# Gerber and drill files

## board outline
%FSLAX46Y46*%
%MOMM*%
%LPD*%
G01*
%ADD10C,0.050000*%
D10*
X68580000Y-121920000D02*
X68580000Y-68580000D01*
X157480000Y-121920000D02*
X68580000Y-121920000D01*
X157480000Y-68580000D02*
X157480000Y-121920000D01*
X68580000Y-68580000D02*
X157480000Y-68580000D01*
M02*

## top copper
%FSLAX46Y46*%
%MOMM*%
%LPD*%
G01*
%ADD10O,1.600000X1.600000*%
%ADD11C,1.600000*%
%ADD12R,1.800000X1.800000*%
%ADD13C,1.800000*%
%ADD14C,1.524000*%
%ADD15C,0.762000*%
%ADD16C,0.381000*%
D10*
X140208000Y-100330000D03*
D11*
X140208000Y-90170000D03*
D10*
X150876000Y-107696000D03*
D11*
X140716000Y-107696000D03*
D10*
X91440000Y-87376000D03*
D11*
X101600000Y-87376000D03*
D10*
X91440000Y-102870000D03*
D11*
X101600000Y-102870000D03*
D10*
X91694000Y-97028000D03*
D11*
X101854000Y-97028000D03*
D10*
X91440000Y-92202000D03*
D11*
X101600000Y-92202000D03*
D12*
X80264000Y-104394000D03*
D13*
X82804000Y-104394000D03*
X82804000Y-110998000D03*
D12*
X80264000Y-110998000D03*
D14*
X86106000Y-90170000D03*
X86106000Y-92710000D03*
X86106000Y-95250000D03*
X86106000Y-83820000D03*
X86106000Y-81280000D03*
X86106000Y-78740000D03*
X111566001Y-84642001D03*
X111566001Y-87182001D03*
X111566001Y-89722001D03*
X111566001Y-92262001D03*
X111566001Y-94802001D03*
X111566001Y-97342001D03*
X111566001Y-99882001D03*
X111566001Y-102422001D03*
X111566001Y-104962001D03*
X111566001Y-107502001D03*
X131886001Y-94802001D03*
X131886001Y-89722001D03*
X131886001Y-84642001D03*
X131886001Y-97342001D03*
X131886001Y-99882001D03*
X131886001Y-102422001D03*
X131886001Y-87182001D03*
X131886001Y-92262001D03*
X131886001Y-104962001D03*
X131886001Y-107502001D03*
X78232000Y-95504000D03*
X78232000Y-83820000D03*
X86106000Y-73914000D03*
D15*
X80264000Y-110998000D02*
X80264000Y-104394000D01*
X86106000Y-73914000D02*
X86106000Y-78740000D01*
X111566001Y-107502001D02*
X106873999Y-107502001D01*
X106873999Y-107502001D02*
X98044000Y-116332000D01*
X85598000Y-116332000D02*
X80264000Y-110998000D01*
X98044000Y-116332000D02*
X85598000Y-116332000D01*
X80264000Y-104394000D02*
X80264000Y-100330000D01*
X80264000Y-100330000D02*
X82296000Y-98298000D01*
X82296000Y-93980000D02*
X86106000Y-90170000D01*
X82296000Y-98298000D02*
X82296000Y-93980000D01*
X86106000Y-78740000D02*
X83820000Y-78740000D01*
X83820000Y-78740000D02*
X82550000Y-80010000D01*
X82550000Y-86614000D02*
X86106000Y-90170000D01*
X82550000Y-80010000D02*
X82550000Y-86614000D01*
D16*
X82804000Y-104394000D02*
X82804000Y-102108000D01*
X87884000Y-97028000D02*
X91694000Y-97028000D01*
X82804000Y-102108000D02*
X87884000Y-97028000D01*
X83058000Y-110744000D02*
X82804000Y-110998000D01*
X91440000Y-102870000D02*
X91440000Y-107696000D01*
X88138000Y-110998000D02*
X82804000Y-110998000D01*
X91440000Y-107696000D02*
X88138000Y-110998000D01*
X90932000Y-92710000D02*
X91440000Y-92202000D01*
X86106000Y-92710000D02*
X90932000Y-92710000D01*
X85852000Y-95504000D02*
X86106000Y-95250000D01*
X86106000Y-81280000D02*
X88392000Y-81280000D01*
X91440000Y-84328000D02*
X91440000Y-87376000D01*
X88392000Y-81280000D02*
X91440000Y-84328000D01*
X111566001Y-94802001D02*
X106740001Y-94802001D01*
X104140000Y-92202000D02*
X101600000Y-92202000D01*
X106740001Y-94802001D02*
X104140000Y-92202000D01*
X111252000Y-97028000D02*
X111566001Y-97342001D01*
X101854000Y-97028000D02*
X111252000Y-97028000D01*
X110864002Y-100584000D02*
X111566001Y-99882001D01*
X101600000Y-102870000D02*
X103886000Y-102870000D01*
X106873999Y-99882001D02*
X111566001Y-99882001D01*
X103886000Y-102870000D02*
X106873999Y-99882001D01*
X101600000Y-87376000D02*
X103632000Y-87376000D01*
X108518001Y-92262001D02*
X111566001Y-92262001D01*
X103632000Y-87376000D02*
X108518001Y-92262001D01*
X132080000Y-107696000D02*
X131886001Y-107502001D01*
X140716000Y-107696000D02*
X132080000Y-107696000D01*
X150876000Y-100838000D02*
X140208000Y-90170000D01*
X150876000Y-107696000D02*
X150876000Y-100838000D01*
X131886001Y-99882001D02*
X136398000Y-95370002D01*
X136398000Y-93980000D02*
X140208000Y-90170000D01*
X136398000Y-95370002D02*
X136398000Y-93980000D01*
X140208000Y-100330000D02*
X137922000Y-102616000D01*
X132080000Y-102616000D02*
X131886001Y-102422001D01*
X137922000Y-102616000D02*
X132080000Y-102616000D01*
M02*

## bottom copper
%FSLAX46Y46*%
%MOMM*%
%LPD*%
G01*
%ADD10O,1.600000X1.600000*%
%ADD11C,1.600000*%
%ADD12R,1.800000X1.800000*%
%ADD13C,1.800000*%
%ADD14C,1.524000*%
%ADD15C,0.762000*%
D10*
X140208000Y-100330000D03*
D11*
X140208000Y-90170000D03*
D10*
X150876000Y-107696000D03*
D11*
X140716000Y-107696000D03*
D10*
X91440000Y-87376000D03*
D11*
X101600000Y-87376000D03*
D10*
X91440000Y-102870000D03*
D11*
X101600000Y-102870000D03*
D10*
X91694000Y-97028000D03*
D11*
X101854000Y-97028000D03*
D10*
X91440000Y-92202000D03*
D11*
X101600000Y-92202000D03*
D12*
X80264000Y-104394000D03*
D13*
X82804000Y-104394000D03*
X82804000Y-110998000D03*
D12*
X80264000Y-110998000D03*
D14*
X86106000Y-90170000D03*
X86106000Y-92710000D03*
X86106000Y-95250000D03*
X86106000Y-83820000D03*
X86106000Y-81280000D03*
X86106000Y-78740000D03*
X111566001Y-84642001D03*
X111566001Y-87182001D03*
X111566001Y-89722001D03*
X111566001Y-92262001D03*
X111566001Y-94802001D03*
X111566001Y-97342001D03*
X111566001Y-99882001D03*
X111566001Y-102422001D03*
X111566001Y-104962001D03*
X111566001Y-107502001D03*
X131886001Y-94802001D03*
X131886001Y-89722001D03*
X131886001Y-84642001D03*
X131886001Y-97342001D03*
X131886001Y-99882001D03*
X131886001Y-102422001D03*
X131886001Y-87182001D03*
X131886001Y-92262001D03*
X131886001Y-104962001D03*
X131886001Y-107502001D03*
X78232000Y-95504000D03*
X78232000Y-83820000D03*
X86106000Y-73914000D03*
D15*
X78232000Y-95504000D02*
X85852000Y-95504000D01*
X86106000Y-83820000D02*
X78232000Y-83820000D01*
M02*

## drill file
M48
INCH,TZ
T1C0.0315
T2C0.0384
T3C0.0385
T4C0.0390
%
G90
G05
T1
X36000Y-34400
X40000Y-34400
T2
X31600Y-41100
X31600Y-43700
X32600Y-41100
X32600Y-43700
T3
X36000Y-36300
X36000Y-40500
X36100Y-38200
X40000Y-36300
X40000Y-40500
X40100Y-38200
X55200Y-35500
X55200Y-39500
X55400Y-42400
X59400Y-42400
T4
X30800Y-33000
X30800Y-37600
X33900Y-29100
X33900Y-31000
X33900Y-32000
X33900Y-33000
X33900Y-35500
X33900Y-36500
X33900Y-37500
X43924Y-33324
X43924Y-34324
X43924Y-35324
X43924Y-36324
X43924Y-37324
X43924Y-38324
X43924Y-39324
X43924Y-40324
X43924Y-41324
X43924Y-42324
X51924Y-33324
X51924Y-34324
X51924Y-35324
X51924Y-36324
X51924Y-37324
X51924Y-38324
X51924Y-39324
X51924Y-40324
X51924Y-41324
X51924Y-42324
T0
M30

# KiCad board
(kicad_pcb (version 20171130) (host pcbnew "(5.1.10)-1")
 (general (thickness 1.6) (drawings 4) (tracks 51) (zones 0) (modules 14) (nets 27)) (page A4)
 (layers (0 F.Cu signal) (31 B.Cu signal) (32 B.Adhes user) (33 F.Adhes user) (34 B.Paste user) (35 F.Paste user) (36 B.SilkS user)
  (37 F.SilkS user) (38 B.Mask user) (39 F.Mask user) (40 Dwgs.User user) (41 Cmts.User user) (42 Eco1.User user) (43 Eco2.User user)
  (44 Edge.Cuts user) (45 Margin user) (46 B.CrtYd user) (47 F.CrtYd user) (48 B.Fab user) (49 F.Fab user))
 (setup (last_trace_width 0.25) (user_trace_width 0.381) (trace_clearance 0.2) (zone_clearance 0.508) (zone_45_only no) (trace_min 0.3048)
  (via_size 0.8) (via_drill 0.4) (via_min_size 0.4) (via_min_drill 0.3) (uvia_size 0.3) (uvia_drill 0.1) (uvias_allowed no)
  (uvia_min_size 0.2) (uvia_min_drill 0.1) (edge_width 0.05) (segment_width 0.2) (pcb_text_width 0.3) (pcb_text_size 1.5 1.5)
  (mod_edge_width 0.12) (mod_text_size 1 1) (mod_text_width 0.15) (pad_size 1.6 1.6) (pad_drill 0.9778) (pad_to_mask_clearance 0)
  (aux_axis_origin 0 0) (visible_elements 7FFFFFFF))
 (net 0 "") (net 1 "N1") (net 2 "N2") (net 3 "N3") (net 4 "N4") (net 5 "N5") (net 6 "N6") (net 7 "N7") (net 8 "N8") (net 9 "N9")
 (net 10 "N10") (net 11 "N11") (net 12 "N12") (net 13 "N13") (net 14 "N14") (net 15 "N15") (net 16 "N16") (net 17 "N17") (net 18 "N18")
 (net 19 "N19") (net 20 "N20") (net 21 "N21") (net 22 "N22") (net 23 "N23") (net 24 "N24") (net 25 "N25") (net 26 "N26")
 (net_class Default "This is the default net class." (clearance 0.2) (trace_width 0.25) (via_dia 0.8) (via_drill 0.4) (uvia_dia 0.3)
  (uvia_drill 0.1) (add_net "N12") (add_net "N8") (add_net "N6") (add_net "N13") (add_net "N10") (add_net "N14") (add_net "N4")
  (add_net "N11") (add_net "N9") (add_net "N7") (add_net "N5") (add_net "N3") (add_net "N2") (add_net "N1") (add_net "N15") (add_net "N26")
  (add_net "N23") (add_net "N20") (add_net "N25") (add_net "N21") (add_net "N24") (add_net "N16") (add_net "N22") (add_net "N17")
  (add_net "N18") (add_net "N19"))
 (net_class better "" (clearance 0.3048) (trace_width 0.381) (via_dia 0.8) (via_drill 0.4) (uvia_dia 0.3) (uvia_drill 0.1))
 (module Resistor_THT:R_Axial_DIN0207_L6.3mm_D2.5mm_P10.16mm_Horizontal (layer F.Cu) (at 140.208 90.17 270)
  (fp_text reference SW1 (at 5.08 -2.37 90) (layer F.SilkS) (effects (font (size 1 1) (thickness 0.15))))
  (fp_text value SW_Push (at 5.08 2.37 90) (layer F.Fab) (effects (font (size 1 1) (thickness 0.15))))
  (pad 2 thru_hole oval (at 10.16 0 270) (size 1.6 1.6) (drill 0.9778) (layers *.Cu *.Mask) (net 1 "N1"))
  (pad 1 thru_hole circle (at 0 0 270) (size 1.6 1.6) (drill 0.9778) (layers *.Cu *.Mask) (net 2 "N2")))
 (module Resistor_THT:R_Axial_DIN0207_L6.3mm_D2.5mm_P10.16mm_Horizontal (layer F.Cu) (at 140.716 107.696)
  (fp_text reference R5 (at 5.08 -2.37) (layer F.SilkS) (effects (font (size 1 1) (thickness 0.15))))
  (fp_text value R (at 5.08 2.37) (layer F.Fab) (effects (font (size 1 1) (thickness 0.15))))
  (pad 2 thru_hole oval (at 10.16 0) (size 1.6 1.6) (drill 0.9778) (layers *.Cu *.Mask) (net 2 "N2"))
  (pad 1 thru_hole circle (at 0 0) (size 1.6 1.6) (drill 0.9778) (layers *.Cu *.Mask) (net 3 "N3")))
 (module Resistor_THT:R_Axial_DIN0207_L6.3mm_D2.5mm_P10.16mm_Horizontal (layer F.Cu) (at 101.6 87.376 180)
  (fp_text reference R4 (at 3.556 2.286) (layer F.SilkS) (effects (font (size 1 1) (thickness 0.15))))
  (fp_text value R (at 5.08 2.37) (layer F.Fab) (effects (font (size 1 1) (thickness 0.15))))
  (pad 2 thru_hole oval (at 10.16 0 180) (size 1.6 1.6) (drill 0.8) (layers *.Cu *.Mask) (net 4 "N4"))
  (pad 1 thru_hole circle (at 0 0 180) (size 1.6 1.6) (drill 0.8) (layers *.Cu *.Mask) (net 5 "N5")))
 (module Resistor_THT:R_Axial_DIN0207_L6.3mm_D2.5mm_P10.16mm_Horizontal (layer F.Cu) (at 101.6 102.87 180)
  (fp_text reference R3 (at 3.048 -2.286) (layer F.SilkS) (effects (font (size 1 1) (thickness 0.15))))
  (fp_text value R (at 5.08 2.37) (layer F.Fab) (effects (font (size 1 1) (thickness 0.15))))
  (pad 2 thru_hole oval (at 10.16 0 180) (size 1.6 1.6) (drill 0.9778) (layers *.Cu *.Mask) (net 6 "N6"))
  (pad 1 thru_hole circle (at 0 0 180) (size 1.6 1.6) (drill 0.9778) (layers *.Cu *.Mask) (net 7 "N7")))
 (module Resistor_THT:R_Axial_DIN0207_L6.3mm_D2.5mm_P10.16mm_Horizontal (layer F.Cu) (at 101.854 97.028 180)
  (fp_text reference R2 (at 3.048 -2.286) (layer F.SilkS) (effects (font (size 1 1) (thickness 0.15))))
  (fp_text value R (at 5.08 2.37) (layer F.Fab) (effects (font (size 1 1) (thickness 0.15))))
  (pad 2 thru_hole oval (at 10.16 0 180) (size 1.6 1.6) (drill 0.9778) (layers *.Cu *.Mask) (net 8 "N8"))
  (pad 1 thru_hole circle (at 0 0 180) (size 1.6 1.6) (drill 0.9778) (layers *.Cu *.Mask) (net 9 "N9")))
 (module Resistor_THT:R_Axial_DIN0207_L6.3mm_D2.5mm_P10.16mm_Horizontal (layer F.Cu) (at 101.6 92.202 180)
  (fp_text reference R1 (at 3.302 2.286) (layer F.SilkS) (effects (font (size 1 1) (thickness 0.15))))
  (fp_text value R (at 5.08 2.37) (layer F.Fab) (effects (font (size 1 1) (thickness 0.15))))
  (pad 2 thru_hole oval (at 10.16 0 180) (size 1.6 1.6) (drill 0.9778) (layers *.Cu *.Mask) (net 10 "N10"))
  (pad 1 thru_hole circle (at 0 0 180) (size 1.6 1.6) (drill 0.9778) (layers *.Cu *.Mask) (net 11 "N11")))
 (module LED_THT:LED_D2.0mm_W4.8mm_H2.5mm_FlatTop (layer F.Cu) (at 80.264 104.394)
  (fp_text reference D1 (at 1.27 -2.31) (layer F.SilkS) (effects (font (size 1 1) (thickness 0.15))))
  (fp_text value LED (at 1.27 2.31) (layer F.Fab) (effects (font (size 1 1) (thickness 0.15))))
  (pad 1 thru_hole rect (at 0 0) (size 1.8 1.8) (drill 0.9762) (layers *.Cu *.Mask) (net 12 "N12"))
  (pad 2 thru_hole circle (at 2.54 0) (size 1.8 1.8) (drill 0.9762) (layers *.Cu *.Mask) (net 8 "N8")))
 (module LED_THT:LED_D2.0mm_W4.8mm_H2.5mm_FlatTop (layer F.Cu) (at 80.264 110.998)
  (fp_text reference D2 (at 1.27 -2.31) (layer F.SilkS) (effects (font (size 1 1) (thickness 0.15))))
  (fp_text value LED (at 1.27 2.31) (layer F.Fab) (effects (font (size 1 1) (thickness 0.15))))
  (pad 2 thru_hole circle (at 2.54 0) (size 1.8 1.8) (drill 0.9762) (layers *.Cu *.Mask) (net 6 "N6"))
  (pad 1 thru_hole rect (at 0 0) (size 1.8 1.8) (drill 0.9762) (layers *.Cu *.Mask) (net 12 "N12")))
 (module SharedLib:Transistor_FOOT (layer F.Cu) (at 86.106 92.71 90)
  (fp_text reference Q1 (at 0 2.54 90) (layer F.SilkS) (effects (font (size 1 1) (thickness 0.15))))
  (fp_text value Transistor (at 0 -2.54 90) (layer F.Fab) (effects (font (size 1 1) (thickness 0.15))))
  (pad 3 thru_hole circle (at 2.54 0 90) (size 1.524 1.524) (drill 0.9906) (layers *.Cu *.Mask) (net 12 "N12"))
  (pad 2 thru_hole circle (at 0 0 90) (size 1.524 1.524) (drill 0.9906) (layers *.Cu *.Mask) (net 10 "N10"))
  (pad 1 thru_hole circle (at -2.54 0 90) (size 1.524 1.524) (drill 0.9906) (layers *.Cu *.Mask) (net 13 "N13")))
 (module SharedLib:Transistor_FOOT (layer F.Cu) (at 86.106 81.28 90)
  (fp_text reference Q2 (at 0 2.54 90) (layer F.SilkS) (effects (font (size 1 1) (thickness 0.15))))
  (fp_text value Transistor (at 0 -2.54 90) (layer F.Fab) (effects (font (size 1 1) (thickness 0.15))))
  (pad 1 thru_hole circle (at -2.54 0 90) (size 1.524 1.524) (drill 0.9906) (layers *.Cu *.Mask) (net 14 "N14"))
  (pad 2 thru_hole circle (at 0 0 90) (size 1.524 1.524) (drill 0.9906) (layers *.Cu *.Mask) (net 4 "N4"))
  (pad 3 thru_hole circle (at 2.54 0 90) (size 1.524 1.524) (drill 0.9906) (layers *.Cu *.Mask) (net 12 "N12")))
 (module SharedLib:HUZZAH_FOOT (layer F.Cu) (at 121.726001 96.072001)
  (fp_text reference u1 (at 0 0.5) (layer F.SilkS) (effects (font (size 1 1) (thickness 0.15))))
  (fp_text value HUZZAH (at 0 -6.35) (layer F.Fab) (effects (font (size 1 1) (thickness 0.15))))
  (pad 1 thru_hole circle (at -10.16 -11.43) (size 1.524 1.524) (drill 0.9906) (layers *.Cu *.Mask) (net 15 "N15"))
  (pad 2 thru_hole circle (at -10.16 -8.89) (size 1.524 1.524) (drill 0.9906) (layers *.Cu *.Mask) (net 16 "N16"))
  (pad 3 thru_hole circle (at -10.16 -6.35) (size 1.524 1.524) (drill 0.9906) (layers *.Cu *.Mask) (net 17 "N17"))
  (pad 4 thru_hole circle (at -10.16 -3.81) (size 1.524 1.524) (drill 0.9906) (layers *.Cu *.Mask) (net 5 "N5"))
  (pad 5 thru_hole circle (at -10.16 -1.27) (size 1.524 1.524) (drill 0.9906) (layers *.Cu *.Mask) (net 11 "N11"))
  (pad 6 thru_hole circle (at -10.16 1.27) (size 1.524 1.524) (drill 0.9906) (layers *.Cu *.Mask) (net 9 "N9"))
  (pad 7 thru_hole circle (at -10.16 3.81) (size 1.524 1.524) (drill 0.9906) (layers *.Cu *.Mask) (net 7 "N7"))
  (pad 8 thru_hole circle (at -10.16 6.35) (size 1.524 1.524) (drill 0.9906) (layers *.Cu *.Mask) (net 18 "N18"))
  (pad 9 thru_hole circle (at -10.16 8.89) (size 1.524 1.524) (drill 0.9906) (layers *.Cu *.Mask) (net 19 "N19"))
  (pad 10 thru_hole circle (at -10.16 11.43) (size 1.524 1.524) (drill 0.9906) (layers *.Cu *.Mask) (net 12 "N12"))
  (pad 16 thru_hole circle (at 10.16 -1.27) (size 1.524 1.524) (drill 0.9906) (layers *.Cu *.Mask) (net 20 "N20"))
  (pad 18 thru_hole circle (at 10.16 -6.35) (size 1.524 1.524) (drill 0.9906) (layers *.Cu *.Mask) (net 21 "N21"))
  (pad 20 thru_hole circle (at 10.16 -11.43) (size 1.524 1.524) (drill 0.9906) (layers *.Cu *.Mask) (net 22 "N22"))
  (pad 15 thru_hole circle (at 10.16 1.27) (size 1.524 1.524) (drill 0.9906) (layers *.Cu *.Mask) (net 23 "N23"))
  (pad 14 thru_hole circle (at 10.16 3.81) (size 1.524 1.524) (drill 0.9906) (layers *.Cu *.Mask) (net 2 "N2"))
  (pad 13 thru_hole circle (at 10.16 6.35) (size 1.524 1.524) (drill 0.9906) (layers *.Cu *.Mask) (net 1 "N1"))
  (pad 19 thru_hole circle (at 10.16 -8.89) (size 1.524 1.524) (drill 0.9906) (layers *.Cu *.Mask) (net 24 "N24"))
  (pad 17 thru_hole circle (at 10.16 -3.81) (size 1.524 1.524) (drill 0.9906) (layers *.Cu *.Mask) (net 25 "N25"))
  (pad 12 thru_hole circle (at 10.16 8.89) (size 1.524 1.524) (drill 0.9906) (layers *.Cu *.Mask) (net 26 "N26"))
  (pad 11 thru_hole circle (at 10.16 11.43) (size 1.524 1.524) (drill 0.9906) (layers *.Cu *.Mask) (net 3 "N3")))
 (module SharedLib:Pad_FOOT (layer F.Cu) (at 78.232 95.504)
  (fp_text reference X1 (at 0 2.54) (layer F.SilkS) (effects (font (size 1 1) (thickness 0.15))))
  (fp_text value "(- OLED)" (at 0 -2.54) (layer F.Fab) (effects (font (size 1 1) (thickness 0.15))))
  (pad 1 thru_hole circle (at 0 0) (size 1.524 1.524) (drill 0.9906) (layers *.Cu *.Mask) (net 13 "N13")))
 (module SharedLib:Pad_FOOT (layer F.Cu) (at 78.232 83.82)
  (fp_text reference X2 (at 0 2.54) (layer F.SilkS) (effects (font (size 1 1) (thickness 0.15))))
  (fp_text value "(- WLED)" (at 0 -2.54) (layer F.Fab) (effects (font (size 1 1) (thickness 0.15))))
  (pad 1 thru_hole circle (at 0 0) (size 1.524 1.524) (drill 0.9906) (layers *.Cu *.Mask) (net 14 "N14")))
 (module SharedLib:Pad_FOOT (layer F.Cu) (at 86.106 73.914)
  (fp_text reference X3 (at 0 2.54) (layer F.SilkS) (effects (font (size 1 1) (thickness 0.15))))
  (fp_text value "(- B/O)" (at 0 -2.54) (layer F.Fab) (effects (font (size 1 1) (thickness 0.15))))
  (pad 1 thru_hole circle (at 0 0) (size 1.524 1.524) (drill 0.9906) (layers *.Cu *.Mask) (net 12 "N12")))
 (gr_line (start 68.58 121.92) (end 68.58 68.58) (layer Edge.Cuts) (width 0.05))
 (gr_line (start 157.48 121.92) (end 68.58 121.92) (layer Edge.Cuts) (width 0.05))
 (gr_line (start 157.48 68.58) (end 157.48 121.92) (layer Edge.Cuts) (width 0.05))
 (gr_line (start 68.58 68.58) (end 157.48 68.58) (layer Edge.Cuts) (width 0.05))
 (segment (start 80.264 110.998) (end 80.264 104.394) (width 0.762) (layer F.Cu) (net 12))
 (segment (start 86.106 73.914) (end 86.106 78.74) (width 0.762) (layer F.Cu) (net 12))
 (segment (start 111.566001 107.502001) (end 106.873999 107.502001) (width 0.762) (layer F.Cu) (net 12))
 (segment (start 106.873999 107.502001) (end 98.044 116.332) (width 0.762) (layer F.Cu) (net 12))
 (segment (start 85.598 116.332) (end 80.264 110.998) (width 0.762) (layer F.Cu) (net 12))
 (segment (start 98.044 116.332) (end 85.598 116.332) (width 0.762) (layer F.Cu) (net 12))
 (segment (start 80.264 104.394) (end 80.264 100.33) (width 0.762) (layer F.Cu) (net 12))
 (segment (start 80.264 100.33) (end 82.296 98.298) (width 0.762) (layer F.Cu) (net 12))
 (segment (start 82.296 93.98) (end 86.106 90.17) (width 0.762) (layer F.Cu) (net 12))
 (segment (start 82.296 98.298) (end 82.296 93.98) (width 0.762) (layer F.Cu) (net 12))
 (segment (start 86.106 78.74) (end 83.82 78.74) (width 0.762) (layer F.Cu) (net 12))
 (segment (start 83.82 78.74) (end 82.55 80.01) (width 0.762) (layer F.Cu) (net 12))
 (segment (start 82.55 86.614) (end 86.106 90.17) (width 0.762) (layer F.Cu) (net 12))
 (segment (start 82.55 80.01) (end 82.55 86.614) (width 0.762) (layer F.Cu) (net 12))
 (segment (start 82.804 104.394) (end 82.804 102.108) (width 0.381) (layer F.Cu) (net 8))
 (segment (start 87.884 97.028) (end 91.694 97.028) (width 0.381) (layer F.Cu) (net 8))
 (segment (start 82.804 102.108) (end 87.884 97.028) (width 0.381) (layer F.Cu) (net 8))
 (segment (start 83.058 110.744) (end 82.804 110.998) (width 0.381) (layer F.Cu) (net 6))
 (segment (start 91.44 102.87) (end 91.44 107.696) (width 0.381) (layer F.Cu) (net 6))
 (segment (start 88.138 110.998) (end 82.804 110.998) (width 0.381) (layer F.Cu) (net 6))
 (segment (start 91.44 107.696) (end 88.138 110.998) (width 0.381) (layer F.Cu) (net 6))
 (segment (start 90.932 92.71) (end 91.44 92.202) (width 0.381) (layer F.Cu) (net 10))
 (segment (start 86.106 92.71) (end 90.932 92.71) (width 0.381) (layer F.Cu) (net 10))
 (segment (start 85.852 95.504) (end 86.106 95.25) (width 0.381) (layer F.Cu) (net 13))
 (segment (start 78.232 95.504) (end 85.852 95.504) (width 0.762) (layer B.Cu) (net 13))
 (segment (start 86.106 83.82) (end 78.232 83.82) (width 0.762) (layer B.Cu) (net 14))
 (segment (start 86.106 81.28) (end 88.392 81.28) (width 0.381) (layer F.Cu) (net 4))
 (segment (start 91.44 84.328) (end 91.44 87.376) (width 0.381) (layer F.Cu) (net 4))
 (segment (start 88.392 81.28) (end 91.44 84.328) (width 0.381) (layer F.Cu) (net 4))
 (segment (start 111.566001 94.802001) (end 106.740001 94.802001) (width 0.381) (layer F.Cu) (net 11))
 (segment (start 104.14 92.202) (end 101.6 92.202) (width 0.381) (layer F.Cu) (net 11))
 (segment (start 106.740001 94.802001) (end 104.14 92.202) (width 0.381) (layer F.Cu) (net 11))
 (segment (start 111.252 97.028) (end 111.566001 97.342001) (width 0.381) (layer F.Cu) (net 9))
 (segment (start 101.854 97.028) (end 111.252 97.028) (width 0.381) (layer F.Cu) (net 9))
 (segment (start 110.864002 100.584) (end 111.566001 99.882001) (width 0.381) (layer F.Cu) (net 7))
 (segment (start 101.6 102.87) (end 103.886 102.87) (width 0.381) (layer F.Cu) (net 7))
 (segment (start 106.873999 99.882001) (end 111.566001 99.882001) (width 0.381) (layer F.Cu) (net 7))
 (segment (start 103.886 102.87) (end 106.873999 99.882001) (width 0.381) (layer F.Cu) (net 7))
 (segment (start 101.6 87.376) (end 103.632 87.376) (width 0.381) (layer F.Cu) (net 5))
 (segment (start 108.518001 92.262001) (end 111.566001 92.262001) (width 0.381) (layer F.Cu) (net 5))
 (segment (start 103.632 87.376) (end 108.518001 92.262001) (width 0.381) (layer F.Cu) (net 5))
 (segment (start 132.08 107.696) (end 131.886001 107.502001) (width 0.381) (layer F.Cu) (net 3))
 (segment (start 140.716 107.696) (end 132.08 107.696) (width 0.381) (layer F.Cu) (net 3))
 (segment (start 150.876 100.838) (end 140.208 90.17) (width 0.381) (layer F.Cu) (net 2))
 (segment (start 150.876 107.696) (end 150.876 100.838) (width 0.381) (layer F.Cu) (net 2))
 (segment (start 131.886001 99.882001) (end 136.398 95.370002) (width 0.381) (layer F.Cu) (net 2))
 (segment (start 136.398 93.98) (end 140.208 90.17) (width 0.381) (layer F.Cu) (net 2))
 (segment (start 136.398 95.370002) (end 136.398 93.98) (width 0.381) (layer F.Cu) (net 2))
 (segment (start 140.208 100.33) (end 137.922 102.616) (width 0.381) (layer F.Cu) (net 1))
 (segment (start 132.08 102.616) (end 131.886001 102.422001) (width 0.381) (layer F.Cu) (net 1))
 (segment (start 137.922 102.616) (end 132.08 102.616) (width 0.381) (layer F.Cu) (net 1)))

